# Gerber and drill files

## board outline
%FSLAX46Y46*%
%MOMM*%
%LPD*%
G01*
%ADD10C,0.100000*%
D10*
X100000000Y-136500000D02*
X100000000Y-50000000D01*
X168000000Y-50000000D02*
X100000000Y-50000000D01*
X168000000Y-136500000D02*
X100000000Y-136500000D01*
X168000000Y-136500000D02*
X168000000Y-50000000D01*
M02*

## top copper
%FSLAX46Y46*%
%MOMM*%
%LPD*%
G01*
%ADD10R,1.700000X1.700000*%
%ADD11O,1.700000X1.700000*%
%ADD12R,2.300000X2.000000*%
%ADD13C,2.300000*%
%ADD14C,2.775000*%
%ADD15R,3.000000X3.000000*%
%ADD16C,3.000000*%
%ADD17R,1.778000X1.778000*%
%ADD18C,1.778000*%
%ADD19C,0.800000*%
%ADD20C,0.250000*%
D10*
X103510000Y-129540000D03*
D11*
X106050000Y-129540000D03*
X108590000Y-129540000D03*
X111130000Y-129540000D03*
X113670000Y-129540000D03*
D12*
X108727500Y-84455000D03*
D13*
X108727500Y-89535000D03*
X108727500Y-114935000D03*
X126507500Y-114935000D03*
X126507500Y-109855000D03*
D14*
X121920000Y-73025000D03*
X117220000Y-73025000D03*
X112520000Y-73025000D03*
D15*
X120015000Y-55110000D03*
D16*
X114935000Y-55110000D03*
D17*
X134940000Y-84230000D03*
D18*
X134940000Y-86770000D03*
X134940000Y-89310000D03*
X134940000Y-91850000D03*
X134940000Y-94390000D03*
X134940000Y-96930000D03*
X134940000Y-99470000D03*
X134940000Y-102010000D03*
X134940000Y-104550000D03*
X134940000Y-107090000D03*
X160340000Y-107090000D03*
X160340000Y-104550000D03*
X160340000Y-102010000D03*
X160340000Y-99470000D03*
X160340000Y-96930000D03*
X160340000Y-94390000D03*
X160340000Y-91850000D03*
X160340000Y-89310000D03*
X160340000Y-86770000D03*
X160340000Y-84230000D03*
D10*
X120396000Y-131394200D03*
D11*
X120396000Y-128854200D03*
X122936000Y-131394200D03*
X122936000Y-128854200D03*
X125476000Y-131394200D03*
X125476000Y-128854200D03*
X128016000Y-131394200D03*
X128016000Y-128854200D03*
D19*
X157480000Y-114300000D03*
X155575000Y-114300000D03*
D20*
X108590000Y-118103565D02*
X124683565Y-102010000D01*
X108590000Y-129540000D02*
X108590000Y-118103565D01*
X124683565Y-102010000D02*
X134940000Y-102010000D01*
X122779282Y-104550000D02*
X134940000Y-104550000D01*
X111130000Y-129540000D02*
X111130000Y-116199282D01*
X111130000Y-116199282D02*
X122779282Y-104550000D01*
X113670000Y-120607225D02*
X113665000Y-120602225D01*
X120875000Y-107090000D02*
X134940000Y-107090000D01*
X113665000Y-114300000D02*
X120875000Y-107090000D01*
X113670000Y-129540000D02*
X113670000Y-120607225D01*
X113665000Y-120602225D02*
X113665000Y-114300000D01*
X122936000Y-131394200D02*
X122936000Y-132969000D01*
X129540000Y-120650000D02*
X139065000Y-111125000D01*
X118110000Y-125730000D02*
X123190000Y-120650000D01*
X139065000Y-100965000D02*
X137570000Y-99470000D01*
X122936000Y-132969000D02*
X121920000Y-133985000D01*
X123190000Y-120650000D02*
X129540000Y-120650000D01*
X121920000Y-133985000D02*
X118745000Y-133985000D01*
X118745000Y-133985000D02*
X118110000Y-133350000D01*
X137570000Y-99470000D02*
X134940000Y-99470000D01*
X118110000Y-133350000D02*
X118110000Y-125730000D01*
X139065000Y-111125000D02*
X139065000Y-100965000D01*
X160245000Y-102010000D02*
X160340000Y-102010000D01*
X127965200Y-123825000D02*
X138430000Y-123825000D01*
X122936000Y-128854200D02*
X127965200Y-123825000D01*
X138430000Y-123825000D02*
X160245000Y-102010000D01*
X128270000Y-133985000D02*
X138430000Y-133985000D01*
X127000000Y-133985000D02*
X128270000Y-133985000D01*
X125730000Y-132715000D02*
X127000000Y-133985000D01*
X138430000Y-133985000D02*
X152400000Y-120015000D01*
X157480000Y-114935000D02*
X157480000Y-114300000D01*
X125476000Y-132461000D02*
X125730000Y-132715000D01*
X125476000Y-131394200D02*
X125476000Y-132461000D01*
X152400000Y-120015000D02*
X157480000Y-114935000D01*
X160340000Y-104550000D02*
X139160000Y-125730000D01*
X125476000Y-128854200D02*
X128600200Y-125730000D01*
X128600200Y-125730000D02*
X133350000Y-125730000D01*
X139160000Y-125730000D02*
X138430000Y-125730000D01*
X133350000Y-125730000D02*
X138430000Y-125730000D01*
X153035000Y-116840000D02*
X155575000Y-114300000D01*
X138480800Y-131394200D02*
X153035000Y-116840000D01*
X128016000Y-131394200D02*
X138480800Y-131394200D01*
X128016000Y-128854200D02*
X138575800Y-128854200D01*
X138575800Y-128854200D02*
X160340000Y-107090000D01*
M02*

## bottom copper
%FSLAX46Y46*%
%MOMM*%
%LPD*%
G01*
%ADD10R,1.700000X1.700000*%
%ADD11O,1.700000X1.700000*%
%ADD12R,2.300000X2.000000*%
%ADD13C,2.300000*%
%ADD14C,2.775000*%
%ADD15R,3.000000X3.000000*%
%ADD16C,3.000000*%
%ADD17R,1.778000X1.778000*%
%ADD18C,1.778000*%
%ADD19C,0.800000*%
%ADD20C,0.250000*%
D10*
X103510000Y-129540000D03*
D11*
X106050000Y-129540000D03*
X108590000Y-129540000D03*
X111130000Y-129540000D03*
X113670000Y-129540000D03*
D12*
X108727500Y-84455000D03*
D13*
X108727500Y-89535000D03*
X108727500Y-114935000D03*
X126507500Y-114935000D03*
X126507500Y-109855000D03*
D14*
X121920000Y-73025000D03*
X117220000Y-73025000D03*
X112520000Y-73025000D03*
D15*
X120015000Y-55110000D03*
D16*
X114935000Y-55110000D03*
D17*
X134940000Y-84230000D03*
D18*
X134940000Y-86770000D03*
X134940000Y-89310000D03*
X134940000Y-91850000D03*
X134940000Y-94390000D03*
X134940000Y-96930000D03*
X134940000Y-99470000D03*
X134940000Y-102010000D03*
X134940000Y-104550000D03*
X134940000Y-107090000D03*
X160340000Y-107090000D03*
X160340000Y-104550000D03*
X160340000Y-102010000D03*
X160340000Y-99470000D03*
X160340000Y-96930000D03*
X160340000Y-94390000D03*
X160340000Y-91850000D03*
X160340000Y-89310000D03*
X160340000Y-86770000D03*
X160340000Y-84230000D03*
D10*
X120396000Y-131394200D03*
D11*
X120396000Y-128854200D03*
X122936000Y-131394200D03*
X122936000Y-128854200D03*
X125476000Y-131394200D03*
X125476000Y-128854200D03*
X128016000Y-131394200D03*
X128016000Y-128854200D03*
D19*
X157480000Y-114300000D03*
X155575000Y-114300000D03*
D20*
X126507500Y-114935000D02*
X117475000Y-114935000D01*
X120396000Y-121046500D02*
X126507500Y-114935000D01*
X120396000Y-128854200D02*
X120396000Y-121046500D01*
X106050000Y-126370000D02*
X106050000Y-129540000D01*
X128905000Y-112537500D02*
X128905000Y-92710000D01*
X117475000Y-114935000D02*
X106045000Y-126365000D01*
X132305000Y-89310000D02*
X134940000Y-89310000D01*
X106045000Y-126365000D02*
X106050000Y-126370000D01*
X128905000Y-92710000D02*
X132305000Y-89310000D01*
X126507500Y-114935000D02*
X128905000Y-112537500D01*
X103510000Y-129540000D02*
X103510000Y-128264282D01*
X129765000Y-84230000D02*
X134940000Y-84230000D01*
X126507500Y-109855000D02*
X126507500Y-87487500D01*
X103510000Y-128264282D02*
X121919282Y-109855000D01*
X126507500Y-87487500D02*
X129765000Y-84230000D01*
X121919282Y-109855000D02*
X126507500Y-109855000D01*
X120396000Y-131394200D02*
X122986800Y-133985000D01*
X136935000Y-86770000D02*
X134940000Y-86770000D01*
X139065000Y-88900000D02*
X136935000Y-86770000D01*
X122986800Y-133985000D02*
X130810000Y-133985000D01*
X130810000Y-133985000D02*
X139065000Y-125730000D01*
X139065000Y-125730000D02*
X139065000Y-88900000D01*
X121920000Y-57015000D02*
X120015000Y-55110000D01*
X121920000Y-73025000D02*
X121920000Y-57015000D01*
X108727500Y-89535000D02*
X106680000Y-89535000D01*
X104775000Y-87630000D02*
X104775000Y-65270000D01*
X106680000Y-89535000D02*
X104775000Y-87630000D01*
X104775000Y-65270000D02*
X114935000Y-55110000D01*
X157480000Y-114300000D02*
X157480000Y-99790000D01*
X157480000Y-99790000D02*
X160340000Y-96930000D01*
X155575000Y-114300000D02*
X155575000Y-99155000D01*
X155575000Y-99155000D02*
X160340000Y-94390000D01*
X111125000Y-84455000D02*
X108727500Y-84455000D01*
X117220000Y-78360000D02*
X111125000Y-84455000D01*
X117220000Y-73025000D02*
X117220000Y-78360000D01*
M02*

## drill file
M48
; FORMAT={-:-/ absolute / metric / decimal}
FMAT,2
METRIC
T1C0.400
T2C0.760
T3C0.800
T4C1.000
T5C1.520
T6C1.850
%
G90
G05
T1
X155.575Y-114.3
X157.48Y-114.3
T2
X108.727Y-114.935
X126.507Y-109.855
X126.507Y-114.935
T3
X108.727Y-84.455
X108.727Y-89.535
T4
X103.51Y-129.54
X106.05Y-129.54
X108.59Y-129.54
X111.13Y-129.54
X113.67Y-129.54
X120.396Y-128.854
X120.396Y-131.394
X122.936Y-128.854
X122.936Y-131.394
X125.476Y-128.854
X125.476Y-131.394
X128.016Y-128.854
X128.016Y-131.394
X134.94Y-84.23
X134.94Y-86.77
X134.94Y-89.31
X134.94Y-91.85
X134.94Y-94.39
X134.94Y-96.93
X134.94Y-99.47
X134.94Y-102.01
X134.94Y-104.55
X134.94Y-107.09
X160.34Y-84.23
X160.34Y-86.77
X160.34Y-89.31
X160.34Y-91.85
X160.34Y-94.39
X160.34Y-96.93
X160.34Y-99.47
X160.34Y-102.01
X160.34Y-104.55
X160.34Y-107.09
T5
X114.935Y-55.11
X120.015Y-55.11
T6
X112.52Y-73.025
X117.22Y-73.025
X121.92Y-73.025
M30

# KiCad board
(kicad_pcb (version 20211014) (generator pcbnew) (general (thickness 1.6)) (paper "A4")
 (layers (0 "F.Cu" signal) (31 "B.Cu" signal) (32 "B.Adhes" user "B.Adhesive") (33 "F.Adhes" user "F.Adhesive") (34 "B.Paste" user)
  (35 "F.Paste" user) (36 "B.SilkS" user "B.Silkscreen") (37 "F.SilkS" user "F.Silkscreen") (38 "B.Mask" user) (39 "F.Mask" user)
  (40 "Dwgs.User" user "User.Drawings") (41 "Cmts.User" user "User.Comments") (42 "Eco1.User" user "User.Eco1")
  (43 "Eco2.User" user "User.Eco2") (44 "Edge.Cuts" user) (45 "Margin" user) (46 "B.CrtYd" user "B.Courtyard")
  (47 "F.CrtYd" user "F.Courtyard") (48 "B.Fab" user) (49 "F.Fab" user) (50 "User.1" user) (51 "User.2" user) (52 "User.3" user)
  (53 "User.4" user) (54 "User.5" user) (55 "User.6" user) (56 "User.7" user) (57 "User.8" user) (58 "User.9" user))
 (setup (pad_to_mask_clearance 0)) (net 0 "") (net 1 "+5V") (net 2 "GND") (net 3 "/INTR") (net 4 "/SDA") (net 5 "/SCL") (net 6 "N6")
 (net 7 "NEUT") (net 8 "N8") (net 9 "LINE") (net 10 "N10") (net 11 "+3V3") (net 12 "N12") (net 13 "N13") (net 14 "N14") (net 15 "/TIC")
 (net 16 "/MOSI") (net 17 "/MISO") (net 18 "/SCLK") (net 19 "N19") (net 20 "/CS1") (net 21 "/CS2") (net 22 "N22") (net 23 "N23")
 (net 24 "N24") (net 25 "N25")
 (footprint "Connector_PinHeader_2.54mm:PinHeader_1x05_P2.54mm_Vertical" (layer "F.Cu") (at 103.51 129.54 90)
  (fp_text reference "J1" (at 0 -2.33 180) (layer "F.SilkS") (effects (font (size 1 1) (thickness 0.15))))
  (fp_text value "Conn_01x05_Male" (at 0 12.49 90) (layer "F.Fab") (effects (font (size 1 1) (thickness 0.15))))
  (pad "1" thru_hole rect locked (at 0 0 90) (size 1.7 1.7) (drill 1) (layers *.Cu *.Mask) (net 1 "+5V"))
  (pad "2" thru_hole oval locked (at 0 2.54 90) (size 1.7 1.7) (drill 1) (layers *.Cu *.Mask) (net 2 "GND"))
  (pad "3" thru_hole oval locked (at 0 5.08 90) (size 1.7 1.7) (drill 1) (layers *.Cu *.Mask) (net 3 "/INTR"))
  (pad "4" thru_hole oval locked (at 0 7.62 90) (size 1.7 1.7) (drill 1) (layers *.Cu *.Mask) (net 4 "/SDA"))
  (pad "5" thru_hole oval locked (at 0 10.16 90) (size 1.7 1.7) (drill 1) (layers *.Cu *.Mask) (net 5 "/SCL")))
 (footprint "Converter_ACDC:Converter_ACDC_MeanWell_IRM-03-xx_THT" (layer "F.Cu") (at 108.7275 84.455)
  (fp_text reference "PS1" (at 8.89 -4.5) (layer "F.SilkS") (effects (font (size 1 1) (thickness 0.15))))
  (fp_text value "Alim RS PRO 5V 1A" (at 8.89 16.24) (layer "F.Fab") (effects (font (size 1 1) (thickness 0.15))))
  (pad "1" thru_hole rect locked (at 0 0) (size 2.3 2) (drill 0.8) (layers *.Cu *.Mask) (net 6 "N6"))
  (pad "3" thru_hole circle locked (at 0 5.08) (size 2.3 2.3) (drill 0.8) (layers *.Cu *.Mask) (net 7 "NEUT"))
  (pad "5" thru_hole circle locked (at 0 30.48) (size 2.3 2.3) (drill 0.76) (layers *.Cu *.Mask) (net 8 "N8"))
  (pad "14" thru_hole circle locked (at 17.78 30.48) (size 2.3 2.3) (drill 0.76) (layers *.Cu *.Mask) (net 2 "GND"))
  (pad "16" thru_hole circle locked (at 17.78 25.4) (size 2.3 2.3) (drill 0.76) (layers *.Cu *.Mask) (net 1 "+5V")))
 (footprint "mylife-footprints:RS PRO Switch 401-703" (layer "F.Cu") (at 121.92 73.025 90)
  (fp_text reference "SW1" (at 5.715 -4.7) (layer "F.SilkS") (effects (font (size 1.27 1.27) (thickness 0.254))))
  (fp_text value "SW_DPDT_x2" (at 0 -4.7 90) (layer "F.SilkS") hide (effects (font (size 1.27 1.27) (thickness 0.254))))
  (pad "1" thru_hole circle (at 0 0 90) (size 2.775 2.775) (drill 1.85) (layers *.Cu *.Mask) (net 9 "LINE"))
  (pad "2" thru_hole circle (at 0 -4.7 90) (size 2.775 2.775) (drill 1.85) (layers *.Cu *.Mask) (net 6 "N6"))
  (pad "3" thru_hole circle (at 0 -9.4 90) (size 2.775 2.775) (drill 1.85) (layers *.Cu *.Mask) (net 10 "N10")))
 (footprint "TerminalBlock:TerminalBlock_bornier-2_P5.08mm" (layer "F.Cu") (at 120.015 55.11 180)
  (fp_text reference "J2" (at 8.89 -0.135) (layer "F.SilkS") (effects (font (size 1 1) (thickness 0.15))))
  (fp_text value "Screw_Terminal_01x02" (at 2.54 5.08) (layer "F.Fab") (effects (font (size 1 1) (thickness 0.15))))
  (pad "1" thru_hole rect locked (at 0 0 180) (size 3 3) (drill 1.52) (layers *.Cu *.Mask) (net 9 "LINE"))
  (pad "2" thru_hole circle locked (at 5.08 0 180) (size 3 3) (drill 1.52) (layers *.Cu *.Mask) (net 7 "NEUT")))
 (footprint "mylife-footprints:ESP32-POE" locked (layer "F.Cu") (at 147.68 94.26)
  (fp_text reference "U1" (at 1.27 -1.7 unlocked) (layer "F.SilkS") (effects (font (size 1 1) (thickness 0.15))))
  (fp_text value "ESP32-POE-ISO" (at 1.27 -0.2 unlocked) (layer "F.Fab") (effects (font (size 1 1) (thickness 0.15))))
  (pad "1" thru_hole rect locked (at -12.74 -10.03 270) (size 1.778 1.778) (drill 1) (layers *.Cu *.Mask) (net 1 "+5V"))
  (pad "2" thru_hole circle locked (at -12.74 -7.49 270) (size 1.778 1.778) (drill 1) (layers *.Cu *.Mask) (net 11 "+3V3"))
  (pad "3" thru_hole circle locked (at -12.74 -4.95 270) (size 1.778 1.778) (drill 1) (layers *.Cu *.Mask) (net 2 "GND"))
  (pad "4" thru_hole circle locked (at -12.74 -2.41 270) (size 1.778 1.778) (drill 1) (layers *.Cu *.Mask) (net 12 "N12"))
  (pad "5" thru_hole circle locked (at -12.74 0.13 270) (size 1.778 1.778) (drill 1) (layers *.Cu *.Mask) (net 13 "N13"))
  (pad "6" thru_hole circle locked (at -12.74 2.67 270) (size 1.778 1.778) (drill 1) (layers *.Cu *.Mask) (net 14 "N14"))
  (pad "7" thru_hole circle locked (at -12.74 5.21 270) (size 1.778 1.778) (drill 1) (layers *.Cu *.Mask) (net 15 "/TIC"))
  (pad "8" thru_hole circle locked (at -12.74 7.75 270) (size 1.778 1.778) (drill 1) (layers *.Cu *.Mask) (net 3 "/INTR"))
  (pad "9" thru_hole circle locked (at -12.74 10.29 270) (size 1.778 1.778) (drill 1) (layers *.Cu *.Mask) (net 4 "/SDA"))
  (pad "10" thru_hole circle locked (at -12.74 12.83 270) (size 1.778 1.778) (drill 1) (layers *.Cu *.Mask) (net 5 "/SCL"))
  (pad "11" thru_hole circle locked (at 12.66 12.83 270) (size 1.778 1.778) (drill 1) (layers *.Cu *.Mask) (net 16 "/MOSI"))
  (pad "12" thru_hole circle locked (at 12.66 10.29 270) (size 1.778 1.778) (drill 1) (layers *.Cu *.Mask) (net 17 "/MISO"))
  (pad "13" thru_hole circle locked (at 12.66 7.75 270) (size 1.778 1.778) (drill 1) (layers *.Cu *.Mask) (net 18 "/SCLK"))
  (pad "14" thru_hole circle locked (at 12.66 5.21 270) (size 1.778 1.778) (drill 1) (layers *.Cu *.Mask) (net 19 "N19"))
  (pad "15" thru_hole circle locked (at 12.66 2.67 270) (size 1.778 1.778) (drill 1) (layers *.Cu *.Mask) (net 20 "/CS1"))
  (pad "16" thru_hole circle locked (at 12.66 0.13 270) (size 1.778 1.778) (drill 1) (layers *.Cu *.Mask) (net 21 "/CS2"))
  (pad "17" thru_hole circle locked (at 12.66 -2.41 270) (size 1.778 1.778) (drill 1) (layers *.Cu *.Mask) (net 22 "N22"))
  (pad "18" thru_hole circle locked (at 12.66 -4.95 270) (size 1.778 1.778) (drill 1) (layers *.Cu *.Mask) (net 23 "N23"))
  (pad "19" thru_hole circle locked (at 12.66 -7.49 270) (size 1.778 1.778) (drill 1) (layers *.Cu *.Mask) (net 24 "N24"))
  (pad "20" thru_hole circle locked (at 12.66 -10.03 270) (size 1.778 1.778) (drill 1) (layers *.Cu *.Mask) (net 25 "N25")))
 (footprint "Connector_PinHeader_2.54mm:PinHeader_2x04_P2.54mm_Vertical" (layer "F.Cu") (at 120.396 131.3942 90)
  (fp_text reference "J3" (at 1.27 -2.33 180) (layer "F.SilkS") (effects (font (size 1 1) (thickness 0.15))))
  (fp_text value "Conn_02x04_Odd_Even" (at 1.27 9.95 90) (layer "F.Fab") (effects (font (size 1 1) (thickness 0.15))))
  (pad "1" thru_hole rect locked (at 0 0 90) (size 1.7 1.7) (drill 1) (layers *.Cu *.Mask) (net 11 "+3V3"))
  (pad "2" thru_hole oval locked (at 2.54 0 90) (size 1.7 1.7) (drill 1) (layers *.Cu *.Mask) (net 2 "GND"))
  (pad "3" thru_hole oval locked (at 0 2.54 90) (size 1.7 1.7) (drill 1) (layers *.Cu *.Mask) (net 15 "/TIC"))
  (pad "4" thru_hole oval locked (at 2.54 2.54 90) (size 1.7 1.7) (drill 1) (layers *.Cu *.Mask) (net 18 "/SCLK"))
  (pad "5" thru_hole oval locked (at 0 5.08 90) (size 1.7 1.7) (drill 1) (layers *.Cu *.Mask) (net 20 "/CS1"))
  (pad "6" thru_hole oval locked (at 2.54 5.08 90) (size 1.7 1.7) (drill 1) (layers *.Cu *.Mask) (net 17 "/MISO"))
  (pad "7" thru_hole oval locked (at 0 7.62 90) (size 1.7 1.7) (drill 1) (layers *.Cu *.Mask) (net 21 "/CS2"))
  (pad "8" thru_hole oval locked (at 2.54 7.62 90) (size 1.7 1.7) (drill 1) (layers *.Cu *.Mask) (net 16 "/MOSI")))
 (gr_line locked (start 100 136.5) (end 100 50) (layer "Edge.Cuts") (width 0.1))
 (gr_line locked (start 168 50) (end 100 50) (layer "Edge.Cuts") (width 0.1))
 (gr_line locked (start 168 136.5) (end 100 136.5) (layer "Edge.Cuts") (width 0.1))
 (gr_line locked (start 168 136.5) (end 168 50) (layer "Edge.Cuts") (width 0.1))
 (segment (start 126.5075 114.935) (end 117.475 114.935) (width 0.25) (layer "B.Cu") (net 2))
 (segment (start 120.396 121.0465) (end 126.5075 114.935) (width 0.25) (layer "B.Cu") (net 2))
 (segment (start 120.396 128.8542) (end 120.396 121.0465) (width 0.25) (layer "B.Cu") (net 2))
 (segment (start 106.05 126.37) (end 106.05 129.54) (width 0.25) (layer "B.Cu") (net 2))
 (segment (start 128.905 112.5375) (end 128.905 92.71) (width 0.25) (layer "B.Cu") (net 2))
 (segment (start 117.475 114.935) (end 106.045 126.365) (width 0.25) (layer "B.Cu") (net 2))
 (segment (start 132.305 89.31) (end 134.94 89.31) (width 0.25) (layer "B.Cu") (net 2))
 (segment (start 106.045 126.365) (end 106.05 126.37) (width 0.25) (layer "B.Cu") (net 2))
 (segment (start 128.905 92.71) (end 132.305 89.31) (width 0.25) (layer "B.Cu") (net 2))
 (segment (start 126.5075 114.935) (end 128.905 112.5375) (width 0.25) (layer "B.Cu") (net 2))
 (segment (start 103.51 129.54) (end 103.51 128.264282) (width 0.25) (layer "B.Cu") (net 1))
 (segment (start 129.765 84.23) (end 134.94 84.23) (width 0.25) (layer "B.Cu") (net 1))
 (segment (start 126.5075 109.855) (end 126.5075 87.4875) (width 0.25) (layer "B.Cu") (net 1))
 (segment (start 103.51 128.264282) (end 121.919282 109.855) (width 0.25) (layer "B.Cu") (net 1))
 (segment (start 126.5075 87.4875) (end 129.765 84.23) (width 0.25) (layer "B.Cu") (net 1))
 (segment (start 121.919282 109.855) (end 126.5075 109.855) (width 0.25) (layer "B.Cu") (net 1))
 (segment (start 120.396 131.3942) (end 122.9868 133.985) (width 0.25) (layer "B.Cu") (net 11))
 (segment (start 136.935 86.77) (end 134.94 86.77) (width 0.25) (layer "B.Cu") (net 11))
 (segment (start 139.065 88.9) (end 136.935 86.77) (width 0.25) (layer "B.Cu") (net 11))
 (segment (start 122.9868 133.985) (end 130.81 133.985) (width 0.25) (layer "B.Cu") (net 11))
 (segment (start 130.81 133.985) (end 139.065 125.73) (width 0.25) (layer "B.Cu") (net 11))
 (segment (start 139.065 125.73) (end 139.065 88.9) (width 0.25) (layer "B.Cu") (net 11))
 (segment (start 121.92 57.015) (end 120.015 55.11) (width 0.25) (layer "B.Cu") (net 9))
 (segment (start 121.92 73.025) (end 121.92 57.015) (width 0.25) (layer "B.Cu") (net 9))
 (segment (start 108.7275 89.535) (end 106.68 89.535) (width 0.25) (layer "B.Cu") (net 7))
 (segment (start 104.775 87.63) (end 104.775 65.27) (width 0.25) (layer "B.Cu") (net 7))
 (segment (start 106.68 89.535) (end 104.775 87.63) (width 0.25) (layer "B.Cu") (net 7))
 (segment (start 104.775 65.27) (end 114.935 55.11) (width 0.25) (layer "B.Cu") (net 7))
 (segment (start 108.59 118.103565) (end 124.683565 102.01) (width 0.25) (layer "F.Cu") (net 3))
 (segment (start 108.59 129.54) (end 108.59 118.103565) (width 0.25) (layer "F.Cu") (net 3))
 (segment (start 124.683565 102.01) (end 134.94 102.01) (width 0.25) (layer "F.Cu") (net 3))
 (segment (start 122.779282 104.55) (end 134.94 104.55) (width 0.25) (layer "F.Cu") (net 4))
 (segment (start 111.13 129.54) (end 111.13 116.199282) (width 0.25) (layer "F.Cu") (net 4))
 (segment (start 111.13 116.199282) (end 122.779282 104.55) (width 0.25) (layer "F.Cu") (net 4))
 (segment (start 113.67 120.607225) (end 113.665 120.602225) (width 0.25) (layer "F.Cu") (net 5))
 (segment (start 120.875 107.09) (end 134.94 107.09) (width 0.25) (layer "F.Cu") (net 5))
 (segment (start 113.665 114.3) (end 120.875 107.09) (width 0.25) (layer "F.Cu") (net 5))
 (segment (start 113.67 129.54) (end 113.67 120.607225) (width 0.25) (layer "F.Cu") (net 5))
 (segment (start 113.665 120.602225) (end 113.665 114.3) (width 0.25) (layer "F.Cu") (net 5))
 (segment (start 122.936 131.3942) (end 122.936 132.969) (width 0.25) (layer "F.Cu") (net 15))
 (segment (start 129.54 120.65) (end 139.065 111.125) (width 0.25) (layer "F.Cu") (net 15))
 (segment (start 118.11 125.73) (end 123.19 120.65) (width 0.25) (layer "F.Cu") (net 15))
 (segment (start 139.065 100.965) (end 137.57 99.47) (width 0.25) (layer "F.Cu") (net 15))
 (segment (start 122.936 132.969) (end 121.92 133.985) (width 0.25) (layer "F.Cu") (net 15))
 (segment (start 123.19 120.65) (end 129.54 120.65) (width 0.25) (layer "F.Cu") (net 15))
 (segment (start 121.92 133.985) (end 118.745 133.985) (width 0.25) (layer "F.Cu") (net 15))
 (segment (start 118.745 133.985) (end 118.11 133.35) (width 0.25) (layer "F.Cu") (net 15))
 (segment (start 137.57 99.47) (end 134.94 99.47) (width 0.25) (layer "F.Cu") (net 15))
 (segment (start 118.11 133.35) (end 118.11 125.73) (width 0.25) (layer "F.Cu") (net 15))
 (segment (start 139.065 111.125) (end 139.065 100.965) (width 0.25) (layer "F.Cu") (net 15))
 (segment (start 160.245 102.01) (end 160.34 102.01) (width 0.25) (layer "F.Cu") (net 18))
 (segment (start 127.9652 123.825) (end 138.43 123.825) (width 0.25) (layer "F.Cu") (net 18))
 (segment (start 122.936 128.8542) (end 127.9652 123.825) (width 0.25) (layer "F.Cu") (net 18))
 (segment (start 138.43 123.825) (end 160.245 102.01) (width 0.25) (layer "F.Cu") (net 18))
 (segment (start 128.27 133.985) (end 138.43 133.985) (width 0.25) (layer "F.Cu") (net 20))
 (segment (start 127 133.985) (end 128.27 133.985) (width 0.25) (layer "F.Cu") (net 20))
 (segment (start 125.73 132.715) (end 127 133.985) (width 0.25) (layer "F.Cu") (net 20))
 (segment (start 138.43 133.985) (end 152.4 120.015) (width 0.25) (layer "F.Cu") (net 20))
 (segment (start 157.48 114.935) (end 157.48 114.3) (width 0.25) (layer "F.Cu") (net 20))
 (segment (start 125.476 132.461) (end 125.73 132.715) (width 0.25) (layer "F.Cu") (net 20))
 (segment (start 125.476 131.3942) (end 125.476 132.461) (width 0.25) (layer "F.Cu") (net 20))
 (segment (start 152.4 120.015) (end 157.48 114.935) (width 0.25) (layer "F.Cu") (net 20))
 (via (at 157.48 114.3) (size 0.8) (drill 0.4) (layers "F.Cu" "B.Cu") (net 20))
 (segment (start 157.48 114.3) (end 157.48 99.79) (width 0.25) (layer "B.Cu") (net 20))
 (segment (start 157.48 99.79) (end 160.34 96.93) (width 0.25) (layer "B.Cu") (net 20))
 (segment (start 160.34 104.55) (end 139.16 125.73) (width 0.25) (layer "F.Cu") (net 17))
 (segment (start 125.476 128.8542) (end 128.6002 125.73) (width 0.25) (layer "F.Cu") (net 17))
 (segment (start 128.6002 125.73) (end 133.35 125.73) (width 0.25) (layer "F.Cu") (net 17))
 (segment (start 139.16 125.73) (end 138.43 125.73) (width 0.25) (layer "F.Cu") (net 17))
 (segment (start 133.35 125.73) (end 138.43 125.73) (width 0.25) (layer "F.Cu") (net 17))
 (segment (start 153.035 116.84) (end 155.575 114.3) (width 0.25) (layer "F.Cu") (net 21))
 (segment (start 138.4808 131.3942) (end 153.035 116.84) (width 0.25) (layer "F.Cu") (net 21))
 (segment (start 128.016 131.3942) (end 138.4808 131.3942) (width 0.25) (layer "F.Cu") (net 21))
 (via (at 155.575 114.3) (size 0.8) (drill 0.4) (layers "F.Cu" "B.Cu") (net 21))
 (segment (start 155.575 114.3) (end 155.575 99.155) (width 0.25) (layer "B.Cu") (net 21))
 (segment (start 155.575 99.155) (end 160.34 94.39) (width 0.25) (layer "B.Cu") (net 21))
 (segment (start 128.016 128.8542) (end 138.5758 128.8542) (width 0.25) (layer "F.Cu") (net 16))
 (segment (start 138.5758 128.8542) (end 160.34 107.09) (width 0.25) (layer "F.Cu") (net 16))
 (segment (start 111.125 84.455) (end 108.7275 84.455) (width 0.25) (layer "B.Cu") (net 6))
 (segment (start 117.22 78.36) (end 111.125 84.455) (width 0.25) (layer "B.Cu") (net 6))
 (segment (start 117.22 73.025) (end 117.22 78.36) (width 0.25) (layer "B.Cu") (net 6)))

